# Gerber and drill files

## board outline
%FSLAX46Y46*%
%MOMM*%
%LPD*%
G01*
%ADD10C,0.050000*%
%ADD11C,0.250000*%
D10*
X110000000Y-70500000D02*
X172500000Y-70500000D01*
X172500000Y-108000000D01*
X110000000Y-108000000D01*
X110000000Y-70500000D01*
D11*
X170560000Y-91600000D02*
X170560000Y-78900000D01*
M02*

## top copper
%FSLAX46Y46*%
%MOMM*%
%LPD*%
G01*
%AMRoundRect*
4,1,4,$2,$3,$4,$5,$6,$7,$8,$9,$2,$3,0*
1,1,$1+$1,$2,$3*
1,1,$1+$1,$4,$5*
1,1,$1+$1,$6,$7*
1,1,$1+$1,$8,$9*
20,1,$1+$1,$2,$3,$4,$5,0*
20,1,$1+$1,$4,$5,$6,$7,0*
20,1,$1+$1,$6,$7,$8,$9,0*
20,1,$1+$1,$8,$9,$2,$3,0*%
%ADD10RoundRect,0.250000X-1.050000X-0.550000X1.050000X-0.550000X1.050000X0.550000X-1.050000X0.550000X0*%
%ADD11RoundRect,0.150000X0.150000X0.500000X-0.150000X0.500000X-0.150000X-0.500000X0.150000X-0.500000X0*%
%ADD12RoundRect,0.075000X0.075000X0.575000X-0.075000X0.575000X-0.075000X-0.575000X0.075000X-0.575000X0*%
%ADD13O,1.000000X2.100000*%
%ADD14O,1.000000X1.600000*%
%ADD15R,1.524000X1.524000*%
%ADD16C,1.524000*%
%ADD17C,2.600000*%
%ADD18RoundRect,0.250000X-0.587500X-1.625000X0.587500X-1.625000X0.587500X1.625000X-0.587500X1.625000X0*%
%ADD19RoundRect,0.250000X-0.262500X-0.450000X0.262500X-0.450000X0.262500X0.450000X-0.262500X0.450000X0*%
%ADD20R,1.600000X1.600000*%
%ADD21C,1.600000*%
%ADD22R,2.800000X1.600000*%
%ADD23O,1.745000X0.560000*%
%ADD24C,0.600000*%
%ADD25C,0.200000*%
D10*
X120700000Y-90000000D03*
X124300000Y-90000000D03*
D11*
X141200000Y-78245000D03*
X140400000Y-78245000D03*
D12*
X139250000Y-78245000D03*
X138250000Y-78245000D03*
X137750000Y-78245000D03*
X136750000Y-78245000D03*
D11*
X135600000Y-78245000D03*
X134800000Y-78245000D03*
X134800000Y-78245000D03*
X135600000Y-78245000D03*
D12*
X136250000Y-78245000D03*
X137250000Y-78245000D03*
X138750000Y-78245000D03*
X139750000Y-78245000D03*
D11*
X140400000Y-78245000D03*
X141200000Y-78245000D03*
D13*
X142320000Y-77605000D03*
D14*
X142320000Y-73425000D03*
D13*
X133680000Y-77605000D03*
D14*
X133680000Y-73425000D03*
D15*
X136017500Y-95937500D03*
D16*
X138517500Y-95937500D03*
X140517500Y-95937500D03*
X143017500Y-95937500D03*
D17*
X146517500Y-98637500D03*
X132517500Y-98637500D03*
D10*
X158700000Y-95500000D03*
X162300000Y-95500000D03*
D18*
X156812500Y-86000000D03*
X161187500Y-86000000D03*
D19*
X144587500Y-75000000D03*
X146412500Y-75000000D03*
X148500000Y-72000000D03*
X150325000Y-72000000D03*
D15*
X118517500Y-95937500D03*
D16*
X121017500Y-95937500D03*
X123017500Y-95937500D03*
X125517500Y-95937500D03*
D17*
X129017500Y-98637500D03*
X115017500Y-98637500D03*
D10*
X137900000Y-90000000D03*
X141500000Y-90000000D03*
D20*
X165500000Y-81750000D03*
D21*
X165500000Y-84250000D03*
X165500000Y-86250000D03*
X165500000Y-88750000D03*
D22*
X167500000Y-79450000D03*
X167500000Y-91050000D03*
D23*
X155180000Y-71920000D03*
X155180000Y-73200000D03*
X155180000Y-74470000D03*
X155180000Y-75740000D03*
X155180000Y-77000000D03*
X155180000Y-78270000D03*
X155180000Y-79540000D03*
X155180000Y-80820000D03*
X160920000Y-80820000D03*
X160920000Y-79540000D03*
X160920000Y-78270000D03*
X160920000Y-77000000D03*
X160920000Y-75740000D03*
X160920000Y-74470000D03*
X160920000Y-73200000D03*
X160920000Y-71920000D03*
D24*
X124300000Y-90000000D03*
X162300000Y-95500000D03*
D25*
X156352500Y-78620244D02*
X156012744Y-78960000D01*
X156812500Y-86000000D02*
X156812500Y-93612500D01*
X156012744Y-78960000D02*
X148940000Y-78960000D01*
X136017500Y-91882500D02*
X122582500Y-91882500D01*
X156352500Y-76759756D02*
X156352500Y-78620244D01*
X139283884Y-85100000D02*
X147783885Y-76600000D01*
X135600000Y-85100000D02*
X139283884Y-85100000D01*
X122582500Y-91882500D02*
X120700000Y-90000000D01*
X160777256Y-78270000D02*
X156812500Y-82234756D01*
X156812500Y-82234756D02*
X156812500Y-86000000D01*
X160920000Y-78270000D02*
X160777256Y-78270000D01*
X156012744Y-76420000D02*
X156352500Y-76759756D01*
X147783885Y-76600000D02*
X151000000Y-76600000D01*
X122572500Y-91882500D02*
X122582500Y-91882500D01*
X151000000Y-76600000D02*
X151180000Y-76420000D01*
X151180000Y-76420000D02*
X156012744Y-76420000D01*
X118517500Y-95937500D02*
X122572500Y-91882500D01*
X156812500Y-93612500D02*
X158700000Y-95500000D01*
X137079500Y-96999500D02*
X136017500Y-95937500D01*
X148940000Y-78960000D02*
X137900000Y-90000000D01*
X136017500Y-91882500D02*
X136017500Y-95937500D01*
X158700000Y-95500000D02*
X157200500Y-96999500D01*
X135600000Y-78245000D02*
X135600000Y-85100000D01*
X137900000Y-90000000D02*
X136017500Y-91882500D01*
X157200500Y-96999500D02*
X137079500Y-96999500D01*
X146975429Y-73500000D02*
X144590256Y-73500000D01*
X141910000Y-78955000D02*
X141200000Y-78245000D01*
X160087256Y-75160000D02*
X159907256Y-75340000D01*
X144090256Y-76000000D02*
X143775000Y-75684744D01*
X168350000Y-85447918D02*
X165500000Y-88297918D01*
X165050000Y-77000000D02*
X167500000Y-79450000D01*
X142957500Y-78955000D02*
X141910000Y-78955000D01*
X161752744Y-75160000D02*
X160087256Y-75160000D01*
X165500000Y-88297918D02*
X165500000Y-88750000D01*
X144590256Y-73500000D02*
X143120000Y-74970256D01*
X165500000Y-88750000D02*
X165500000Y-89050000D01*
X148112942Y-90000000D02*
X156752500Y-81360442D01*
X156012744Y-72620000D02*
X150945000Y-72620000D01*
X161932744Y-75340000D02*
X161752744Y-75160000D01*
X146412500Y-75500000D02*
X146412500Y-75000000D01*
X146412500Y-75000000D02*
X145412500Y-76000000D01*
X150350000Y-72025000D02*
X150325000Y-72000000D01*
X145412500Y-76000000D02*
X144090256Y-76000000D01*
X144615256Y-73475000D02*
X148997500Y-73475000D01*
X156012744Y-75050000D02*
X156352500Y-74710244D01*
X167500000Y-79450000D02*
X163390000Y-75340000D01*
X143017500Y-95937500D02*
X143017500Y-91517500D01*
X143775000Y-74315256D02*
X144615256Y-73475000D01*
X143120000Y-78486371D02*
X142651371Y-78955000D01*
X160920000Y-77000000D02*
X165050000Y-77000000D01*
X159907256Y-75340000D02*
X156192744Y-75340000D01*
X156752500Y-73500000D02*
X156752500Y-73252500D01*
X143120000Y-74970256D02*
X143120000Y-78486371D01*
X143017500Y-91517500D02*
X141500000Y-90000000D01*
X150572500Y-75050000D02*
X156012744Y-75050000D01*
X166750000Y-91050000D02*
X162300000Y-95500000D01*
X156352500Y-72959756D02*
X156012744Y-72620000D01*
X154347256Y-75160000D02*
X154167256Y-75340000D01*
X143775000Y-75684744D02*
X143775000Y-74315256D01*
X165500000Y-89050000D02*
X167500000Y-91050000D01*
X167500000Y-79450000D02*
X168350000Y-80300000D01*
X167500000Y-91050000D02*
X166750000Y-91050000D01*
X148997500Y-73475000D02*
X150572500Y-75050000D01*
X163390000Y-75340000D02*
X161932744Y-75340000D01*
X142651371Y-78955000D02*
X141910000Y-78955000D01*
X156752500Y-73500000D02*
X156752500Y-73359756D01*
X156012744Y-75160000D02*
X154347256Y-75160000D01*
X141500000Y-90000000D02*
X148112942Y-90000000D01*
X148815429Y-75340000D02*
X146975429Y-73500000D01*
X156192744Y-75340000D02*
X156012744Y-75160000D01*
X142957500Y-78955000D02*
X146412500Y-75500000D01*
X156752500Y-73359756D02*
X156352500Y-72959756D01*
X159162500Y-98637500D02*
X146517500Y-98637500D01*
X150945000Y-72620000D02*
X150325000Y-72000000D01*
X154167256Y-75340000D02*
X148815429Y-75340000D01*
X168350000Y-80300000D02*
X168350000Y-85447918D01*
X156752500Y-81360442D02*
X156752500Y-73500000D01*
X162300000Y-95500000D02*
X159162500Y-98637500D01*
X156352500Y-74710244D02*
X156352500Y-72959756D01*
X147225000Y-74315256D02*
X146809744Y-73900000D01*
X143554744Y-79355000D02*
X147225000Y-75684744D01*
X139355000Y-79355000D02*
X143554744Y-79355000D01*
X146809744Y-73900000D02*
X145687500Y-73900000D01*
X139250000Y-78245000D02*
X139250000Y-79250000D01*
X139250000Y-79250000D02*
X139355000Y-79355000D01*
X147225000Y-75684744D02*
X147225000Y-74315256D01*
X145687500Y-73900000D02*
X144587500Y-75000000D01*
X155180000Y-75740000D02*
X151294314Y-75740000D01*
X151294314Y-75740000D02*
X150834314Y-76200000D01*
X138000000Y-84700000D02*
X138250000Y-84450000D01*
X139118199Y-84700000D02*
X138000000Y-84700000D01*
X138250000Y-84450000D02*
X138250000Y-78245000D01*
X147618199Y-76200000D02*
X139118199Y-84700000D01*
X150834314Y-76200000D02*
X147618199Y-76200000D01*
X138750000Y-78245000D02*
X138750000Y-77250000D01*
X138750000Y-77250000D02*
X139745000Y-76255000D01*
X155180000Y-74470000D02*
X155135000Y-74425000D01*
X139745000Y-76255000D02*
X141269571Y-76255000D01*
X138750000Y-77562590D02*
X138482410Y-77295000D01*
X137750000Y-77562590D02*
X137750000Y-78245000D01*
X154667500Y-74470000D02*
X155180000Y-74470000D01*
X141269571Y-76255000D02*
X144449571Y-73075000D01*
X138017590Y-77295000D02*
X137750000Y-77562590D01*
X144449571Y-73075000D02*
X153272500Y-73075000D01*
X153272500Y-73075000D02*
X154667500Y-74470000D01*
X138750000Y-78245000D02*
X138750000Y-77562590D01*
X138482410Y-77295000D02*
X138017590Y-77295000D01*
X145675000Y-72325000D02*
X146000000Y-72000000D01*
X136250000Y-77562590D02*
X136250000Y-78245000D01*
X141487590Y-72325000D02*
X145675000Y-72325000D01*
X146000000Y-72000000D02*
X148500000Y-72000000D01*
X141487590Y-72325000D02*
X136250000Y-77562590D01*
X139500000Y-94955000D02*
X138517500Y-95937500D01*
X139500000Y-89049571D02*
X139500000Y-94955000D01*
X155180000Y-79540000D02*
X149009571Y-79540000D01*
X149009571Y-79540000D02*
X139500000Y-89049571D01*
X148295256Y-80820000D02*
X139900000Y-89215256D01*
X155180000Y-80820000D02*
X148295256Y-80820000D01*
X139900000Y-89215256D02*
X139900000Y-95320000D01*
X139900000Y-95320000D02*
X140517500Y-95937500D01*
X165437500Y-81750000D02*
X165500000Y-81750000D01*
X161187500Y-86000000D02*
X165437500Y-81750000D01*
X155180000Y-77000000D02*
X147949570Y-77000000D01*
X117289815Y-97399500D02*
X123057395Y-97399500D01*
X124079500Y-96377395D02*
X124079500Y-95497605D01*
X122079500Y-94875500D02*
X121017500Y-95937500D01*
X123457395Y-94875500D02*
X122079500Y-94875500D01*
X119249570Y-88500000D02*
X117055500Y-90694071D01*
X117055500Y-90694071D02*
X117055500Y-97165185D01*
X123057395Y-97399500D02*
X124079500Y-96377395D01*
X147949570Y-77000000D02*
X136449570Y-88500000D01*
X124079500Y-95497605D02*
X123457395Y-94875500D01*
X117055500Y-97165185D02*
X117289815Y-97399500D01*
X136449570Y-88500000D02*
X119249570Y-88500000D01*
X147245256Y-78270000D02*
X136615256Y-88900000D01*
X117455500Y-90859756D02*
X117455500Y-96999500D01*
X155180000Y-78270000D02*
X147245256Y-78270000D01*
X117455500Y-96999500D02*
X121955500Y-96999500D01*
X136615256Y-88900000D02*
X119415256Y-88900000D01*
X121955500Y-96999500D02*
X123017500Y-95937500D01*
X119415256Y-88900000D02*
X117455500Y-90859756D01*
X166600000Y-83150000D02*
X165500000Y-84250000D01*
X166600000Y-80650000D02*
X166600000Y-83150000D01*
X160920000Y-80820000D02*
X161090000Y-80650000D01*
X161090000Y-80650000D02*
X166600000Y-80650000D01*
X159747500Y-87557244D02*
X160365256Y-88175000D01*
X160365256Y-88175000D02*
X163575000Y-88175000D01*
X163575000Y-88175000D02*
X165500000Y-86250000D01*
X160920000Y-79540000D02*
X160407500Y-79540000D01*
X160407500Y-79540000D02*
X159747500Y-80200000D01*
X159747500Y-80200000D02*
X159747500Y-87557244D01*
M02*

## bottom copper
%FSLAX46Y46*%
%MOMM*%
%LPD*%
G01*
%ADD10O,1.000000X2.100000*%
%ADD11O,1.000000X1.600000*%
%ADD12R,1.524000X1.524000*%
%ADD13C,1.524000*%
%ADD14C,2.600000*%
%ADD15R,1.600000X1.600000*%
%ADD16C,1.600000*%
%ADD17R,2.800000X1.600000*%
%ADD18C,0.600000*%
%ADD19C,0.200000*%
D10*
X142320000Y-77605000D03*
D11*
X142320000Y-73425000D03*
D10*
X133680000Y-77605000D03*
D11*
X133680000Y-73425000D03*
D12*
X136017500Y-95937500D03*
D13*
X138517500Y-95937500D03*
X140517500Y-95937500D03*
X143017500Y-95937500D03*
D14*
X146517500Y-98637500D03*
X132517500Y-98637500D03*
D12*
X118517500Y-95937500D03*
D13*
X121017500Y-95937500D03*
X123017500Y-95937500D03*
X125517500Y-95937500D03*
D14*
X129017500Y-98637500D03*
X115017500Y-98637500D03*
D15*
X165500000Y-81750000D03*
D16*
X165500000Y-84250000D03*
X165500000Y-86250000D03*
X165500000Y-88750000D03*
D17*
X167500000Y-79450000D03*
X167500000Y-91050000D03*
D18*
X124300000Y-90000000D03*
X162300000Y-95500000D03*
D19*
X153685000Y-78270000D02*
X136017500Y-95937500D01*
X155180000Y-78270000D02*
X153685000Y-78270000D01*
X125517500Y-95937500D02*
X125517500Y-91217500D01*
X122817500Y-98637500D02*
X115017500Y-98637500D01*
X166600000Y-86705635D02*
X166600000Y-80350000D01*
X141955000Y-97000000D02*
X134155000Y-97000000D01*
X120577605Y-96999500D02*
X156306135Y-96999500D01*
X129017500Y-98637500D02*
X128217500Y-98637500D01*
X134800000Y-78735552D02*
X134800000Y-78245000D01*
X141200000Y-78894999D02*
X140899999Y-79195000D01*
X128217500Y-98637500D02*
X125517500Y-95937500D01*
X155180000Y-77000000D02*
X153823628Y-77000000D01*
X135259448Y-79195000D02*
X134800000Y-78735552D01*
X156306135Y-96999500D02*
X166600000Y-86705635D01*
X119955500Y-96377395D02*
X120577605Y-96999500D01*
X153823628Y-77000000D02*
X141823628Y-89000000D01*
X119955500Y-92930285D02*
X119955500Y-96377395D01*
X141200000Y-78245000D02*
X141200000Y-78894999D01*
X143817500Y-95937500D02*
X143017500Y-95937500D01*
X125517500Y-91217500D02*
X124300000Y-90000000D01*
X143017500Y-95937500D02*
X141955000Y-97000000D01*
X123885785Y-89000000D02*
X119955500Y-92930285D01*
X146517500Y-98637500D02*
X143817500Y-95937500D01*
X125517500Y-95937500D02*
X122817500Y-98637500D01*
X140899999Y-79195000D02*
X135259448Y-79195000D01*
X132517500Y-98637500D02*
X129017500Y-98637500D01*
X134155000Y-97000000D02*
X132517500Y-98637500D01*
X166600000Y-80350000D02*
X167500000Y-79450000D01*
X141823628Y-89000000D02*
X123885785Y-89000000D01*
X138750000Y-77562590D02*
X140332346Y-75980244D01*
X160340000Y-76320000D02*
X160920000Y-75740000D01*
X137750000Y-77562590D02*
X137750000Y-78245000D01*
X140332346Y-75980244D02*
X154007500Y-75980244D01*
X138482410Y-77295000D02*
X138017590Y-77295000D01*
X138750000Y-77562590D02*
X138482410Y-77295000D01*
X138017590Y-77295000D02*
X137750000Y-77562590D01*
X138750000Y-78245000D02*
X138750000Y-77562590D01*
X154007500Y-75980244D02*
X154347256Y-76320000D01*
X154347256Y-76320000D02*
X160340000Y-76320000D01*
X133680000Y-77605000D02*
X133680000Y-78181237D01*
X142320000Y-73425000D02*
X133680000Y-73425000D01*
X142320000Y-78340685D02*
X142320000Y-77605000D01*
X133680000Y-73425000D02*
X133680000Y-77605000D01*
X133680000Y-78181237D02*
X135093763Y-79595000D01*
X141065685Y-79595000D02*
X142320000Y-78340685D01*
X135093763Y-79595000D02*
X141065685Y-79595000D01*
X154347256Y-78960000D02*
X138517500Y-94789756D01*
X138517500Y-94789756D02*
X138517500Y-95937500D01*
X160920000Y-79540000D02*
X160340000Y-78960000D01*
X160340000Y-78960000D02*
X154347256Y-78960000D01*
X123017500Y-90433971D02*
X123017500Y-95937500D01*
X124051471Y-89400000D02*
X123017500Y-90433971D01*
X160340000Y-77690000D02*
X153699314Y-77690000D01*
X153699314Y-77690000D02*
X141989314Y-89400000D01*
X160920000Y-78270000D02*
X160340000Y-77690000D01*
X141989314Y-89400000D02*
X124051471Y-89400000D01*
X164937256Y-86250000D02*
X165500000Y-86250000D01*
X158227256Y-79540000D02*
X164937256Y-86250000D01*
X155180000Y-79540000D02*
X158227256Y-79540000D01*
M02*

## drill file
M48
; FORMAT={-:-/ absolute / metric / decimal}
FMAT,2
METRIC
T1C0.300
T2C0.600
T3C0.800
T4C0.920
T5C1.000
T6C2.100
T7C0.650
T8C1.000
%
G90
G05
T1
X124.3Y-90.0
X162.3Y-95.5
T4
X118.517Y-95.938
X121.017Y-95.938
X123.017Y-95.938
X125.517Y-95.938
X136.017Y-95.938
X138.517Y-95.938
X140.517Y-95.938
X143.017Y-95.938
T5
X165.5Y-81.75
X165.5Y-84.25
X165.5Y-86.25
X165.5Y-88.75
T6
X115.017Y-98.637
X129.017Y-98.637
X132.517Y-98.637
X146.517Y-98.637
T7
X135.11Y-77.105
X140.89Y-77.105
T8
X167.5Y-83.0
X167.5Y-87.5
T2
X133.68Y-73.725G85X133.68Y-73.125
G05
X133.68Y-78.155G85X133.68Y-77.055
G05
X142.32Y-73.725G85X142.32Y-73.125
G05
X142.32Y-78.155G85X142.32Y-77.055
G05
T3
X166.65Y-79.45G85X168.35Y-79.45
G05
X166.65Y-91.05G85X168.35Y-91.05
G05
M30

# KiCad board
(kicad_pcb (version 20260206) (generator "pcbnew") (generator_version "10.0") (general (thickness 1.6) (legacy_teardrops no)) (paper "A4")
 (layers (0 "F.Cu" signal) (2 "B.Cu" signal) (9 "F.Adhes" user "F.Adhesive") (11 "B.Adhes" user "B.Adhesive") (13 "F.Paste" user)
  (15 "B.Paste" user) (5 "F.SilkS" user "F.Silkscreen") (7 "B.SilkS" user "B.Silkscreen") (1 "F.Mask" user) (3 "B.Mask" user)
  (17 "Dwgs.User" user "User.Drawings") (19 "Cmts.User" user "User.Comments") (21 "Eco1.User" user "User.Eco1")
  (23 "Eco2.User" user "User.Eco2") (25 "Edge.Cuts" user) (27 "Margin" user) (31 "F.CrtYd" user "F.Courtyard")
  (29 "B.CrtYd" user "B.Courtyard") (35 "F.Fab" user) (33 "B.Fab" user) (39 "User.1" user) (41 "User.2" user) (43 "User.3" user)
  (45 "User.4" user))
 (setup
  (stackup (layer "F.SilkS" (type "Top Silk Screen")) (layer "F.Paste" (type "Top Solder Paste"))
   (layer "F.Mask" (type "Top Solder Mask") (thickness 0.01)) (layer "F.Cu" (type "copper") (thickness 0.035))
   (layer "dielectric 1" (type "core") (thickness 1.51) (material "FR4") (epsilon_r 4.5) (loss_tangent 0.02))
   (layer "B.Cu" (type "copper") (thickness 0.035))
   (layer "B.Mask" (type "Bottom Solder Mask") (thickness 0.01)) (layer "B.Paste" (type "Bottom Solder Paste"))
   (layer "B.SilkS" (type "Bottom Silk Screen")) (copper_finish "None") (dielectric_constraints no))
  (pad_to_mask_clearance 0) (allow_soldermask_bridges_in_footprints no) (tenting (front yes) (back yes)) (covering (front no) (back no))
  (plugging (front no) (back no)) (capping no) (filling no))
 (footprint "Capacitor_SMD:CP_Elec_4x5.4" (layer "F.Cu") (at 122.5 90)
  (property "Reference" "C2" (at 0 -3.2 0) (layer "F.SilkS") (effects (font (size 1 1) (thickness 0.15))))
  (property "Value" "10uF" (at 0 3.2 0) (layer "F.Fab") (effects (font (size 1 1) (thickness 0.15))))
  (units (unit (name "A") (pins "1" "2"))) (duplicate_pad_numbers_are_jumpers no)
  (pad "1" smd roundrect (at -1.8 0) (size 2.6 1.6) (layers "F.Cu" "F.Mask" "F.Paste") (roundrect_rratio 0.15625) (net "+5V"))
  (pad "2" smd roundrect (at 1.8 0) (size 2.6 1.6) (layers "F.Cu" "F.Mask" "F.Paste") (roundrect_rratio 0.15625) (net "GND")))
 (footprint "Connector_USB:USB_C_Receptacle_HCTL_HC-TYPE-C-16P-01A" (layer "F.Cu") (at 138 74.5 180)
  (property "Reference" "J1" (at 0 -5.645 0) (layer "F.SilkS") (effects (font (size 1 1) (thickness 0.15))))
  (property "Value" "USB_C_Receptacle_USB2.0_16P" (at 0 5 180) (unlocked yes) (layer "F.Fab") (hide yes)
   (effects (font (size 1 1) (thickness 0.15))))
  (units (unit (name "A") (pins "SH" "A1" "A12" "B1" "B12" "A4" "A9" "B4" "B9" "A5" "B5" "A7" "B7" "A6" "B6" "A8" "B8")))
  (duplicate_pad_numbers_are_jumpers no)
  (pad "" np_thru_hole circle (at -2.89 -2.605 180) (size 0.65 0.65) (drill 0.65) (layers "*.Mask"))
  (pad "" np_thru_hole circle (at 2.89 -2.605 180) (size 0.65 0.65) (drill 0.65) (layers "*.Mask"))
  (pad "A1" smd roundrect (at -3.2 -3.745 180) (size 0.6 1.3) (layers "F.Cu" "F.Mask" "F.Paste") (roundrect_rratio 0.25) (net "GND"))
  (pad "A4" smd roundrect (at -2.4 -3.745 180) (size 0.6 1.3) (layers "F.Cu" "F.Mask" "F.Paste") (roundrect_rratio 0.25) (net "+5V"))
  (pad "A5" smd roundrect (at -1.25 -3.745 180) (size 0.3 1.3) (layers "F.Cu" "F.Mask" "F.Paste") (roundrect_rratio 0.25)
   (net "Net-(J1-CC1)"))
  (pad "A6" smd roundrect (at -0.25 -3.745 180) (size 0.3 1.3) (layers "F.Cu" "F.Mask" "F.Paste") (roundrect_rratio 0.25)
   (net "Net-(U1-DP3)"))
  (pad "A7" smd roundrect (at 0.25 -3.745 180) (size 0.3 1.3) (layers "F.Cu" "F.Mask" "F.Paste") (roundrect_rratio 0.25)
   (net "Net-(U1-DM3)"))
  (pad "A8" smd roundrect (at 1.25 -3.745 180) (size 0.3 1.3) (layers "F.Cu" "F.Mask" "F.Paste") (roundrect_rratio 0.25)
   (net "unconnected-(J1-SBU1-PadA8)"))
  (pad "A9" smd roundrect (at 2.4 -3.745 180) (size 0.6 1.3) (layers "F.Cu" "F.Mask" "F.Paste") (roundrect_rratio 0.25) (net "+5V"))
  (pad "A12" smd roundrect (at 3.2 -3.745 180) (size 0.6 1.3) (layers "F.Cu" "F.Mask" "F.Paste") (roundrect_rratio 0.25) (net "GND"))
  (pad "B1" smd roundrect (at 3.2 -3.745 180) (size 0.6 1.3) (layers "F.Cu" "F.Mask" "F.Paste") (roundrect_rratio 0.25) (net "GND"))
  (pad "B4" smd roundrect (at 2.4 -3.745 180) (size 0.6 1.3) (layers "F.Cu" "F.Mask" "F.Paste") (roundrect_rratio 0.25) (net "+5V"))
  (pad "B5" smd roundrect (at 1.75 -3.745 180) (size 0.3 1.3) (layers "F.Cu" "F.Mask" "F.Paste") (roundrect_rratio 0.25)
   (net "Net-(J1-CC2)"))
  (pad "B6" smd roundrect (at 0.75 -3.745 180) (size 0.3 1.3) (layers "F.Cu" "F.Mask" "F.Paste") (roundrect_rratio 0.25)
   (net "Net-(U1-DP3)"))
  (pad "B7" smd roundrect (at -0.75 -3.745 180) (size 0.3 1.3) (layers "F.Cu" "F.Mask" "F.Paste") (roundrect_rratio 0.25)
   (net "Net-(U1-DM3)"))
  (pad "B8" smd roundrect (at -1.75 -3.745 180) (size 0.3 1.3) (layers "F.Cu" "F.Mask" "F.Paste") (roundrect_rratio 0.25)
   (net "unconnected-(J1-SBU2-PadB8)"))
  (pad "B9" smd roundrect (at -2.4 -3.745 180) (size 0.6 1.3) (layers "F.Cu" "F.Mask" "F.Paste") (roundrect_rratio 0.25) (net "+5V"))
  (pad "B12" smd roundrect (at -3.2 -3.745 180) (size 0.6 1.3) (layers "F.Cu" "F.Mask" "F.Paste") (roundrect_rratio 0.25) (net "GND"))
  (pad "SH" thru_hole oval (at -4.32 -3.105 180) (size 1 2.1) (drill oval 0.6 1.7) (layers "*.Cu" "*.Mask") (remove_unused_layers no)
   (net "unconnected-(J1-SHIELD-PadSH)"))
  (pad "SH" thru_hole oval (at -4.32 1.075 180) (size 1 1.6) (drill oval 0.6 1.2) (layers "*.Cu" "*.Mask") (remove_unused_layers no)
   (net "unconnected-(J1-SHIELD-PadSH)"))
  (pad "SH" thru_hole oval (at 4.32 -3.105 180) (size 1 2.1) (drill oval 0.6 1.7) (layers "*.Cu" "*.Mask") (remove_unused_layers no)
   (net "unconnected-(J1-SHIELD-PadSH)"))
  (pad "SH" thru_hole oval (at 4.32 1.075 180) (size 1 1.6) (drill oval 0.6 1.2) (layers "*.Cu" "*.Mask") (remove_unused_layers no)
   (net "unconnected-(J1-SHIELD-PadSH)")))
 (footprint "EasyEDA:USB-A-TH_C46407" (layer "F.Cu") (at 139.5175 97.2875)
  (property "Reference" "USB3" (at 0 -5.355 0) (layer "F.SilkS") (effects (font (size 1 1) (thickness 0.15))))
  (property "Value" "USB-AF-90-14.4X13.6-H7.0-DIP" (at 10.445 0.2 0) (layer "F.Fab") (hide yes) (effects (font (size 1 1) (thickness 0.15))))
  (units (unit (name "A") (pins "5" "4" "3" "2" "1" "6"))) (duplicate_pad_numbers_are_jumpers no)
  (pad "1" thru_hole rect (at -3.5 -1.35) (size 1.524 1.524) (drill 0.919988) (layers "*.Cu" "*.Mask") (remove_unused_layers no) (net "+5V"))
  (pad "2" thru_hole circle (at -1 -1.35) (size 1.524 1.524) (drill 0.919988) (layers "*.Cu" "*.Mask") (remove_unused_layers no)
   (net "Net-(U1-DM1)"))
  (pad "3" thru_hole circle (at 1 -1.35) (size 1.524 1.524) (drill 0.919988) (layers "*.Cu" "*.Mask") (remove_unused_layers no)
   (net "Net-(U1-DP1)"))
  (pad "4" thru_hole circle (at 3.5 -1.35) (size 1.524 1.524) (drill 0.919988) (layers "*.Cu" "*.Mask") (remove_unused_layers no)
   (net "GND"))
  (pad "5" thru_hole circle (at 7 1.35) (size 2.6 2.6) (drill 2.100022) (layers "*.Cu" "*.Mask") (remove_unused_layers no) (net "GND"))
  (pad "6" thru_hole circle (at -7 1.35) (size 2.6 2.6) (drill 2.100022) (layers "*.Cu" "*.Mask") (remove_unused_layers no) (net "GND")))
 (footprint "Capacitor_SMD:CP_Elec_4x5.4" (layer "F.Cu") (at 160.5 95.5)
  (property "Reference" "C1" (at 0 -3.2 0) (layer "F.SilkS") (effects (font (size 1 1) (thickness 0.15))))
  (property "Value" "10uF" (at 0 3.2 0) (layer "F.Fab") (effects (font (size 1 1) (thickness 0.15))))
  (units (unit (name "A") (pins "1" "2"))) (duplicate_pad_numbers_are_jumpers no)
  (pad "1" smd roundrect (at -1.8 0) (size 2.6 1.6) (layers "F.Cu" "F.Mask" "F.Paste") (roundrect_rratio 0.15625) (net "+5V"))
  (pad "2" smd roundrect (at 1.8 0) (size 2.6 1.6) (layers "F.Cu" "F.Mask" "F.Paste") (roundrect_rratio 0.15625) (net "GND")))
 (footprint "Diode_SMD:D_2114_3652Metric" (layer "F.Cu") (at 159 86)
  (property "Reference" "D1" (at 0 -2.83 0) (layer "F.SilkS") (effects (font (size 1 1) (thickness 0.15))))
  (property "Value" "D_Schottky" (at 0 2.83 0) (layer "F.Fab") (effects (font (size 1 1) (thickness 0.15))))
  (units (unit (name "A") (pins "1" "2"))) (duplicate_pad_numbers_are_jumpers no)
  (pad "1" smd roundrect (at -2.1875 0) (size 1.675 3.75) (layers "F.Cu" "F.Mask" "F.Paste") (roundrect_rratio 0.149254) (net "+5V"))
  (pad "2" smd roundrect (at 2.1875 0) (size 1.675 3.75) (layers "F.Cu" "F.Mask" "F.Paste") (roundrect_rratio 0.149254) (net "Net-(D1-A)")))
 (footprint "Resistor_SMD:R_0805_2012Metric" (layer "F.Cu") (at 145.5 75)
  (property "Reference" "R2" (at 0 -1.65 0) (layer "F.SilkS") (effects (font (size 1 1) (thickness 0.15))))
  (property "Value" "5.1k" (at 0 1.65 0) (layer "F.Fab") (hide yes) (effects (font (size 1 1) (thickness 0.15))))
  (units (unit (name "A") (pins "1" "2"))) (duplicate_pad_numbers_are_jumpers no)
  (pad "1" smd roundrect (at -0.9125 0) (size 1.025 1.4) (layers "F.Cu" "F.Mask" "F.Paste") (roundrect_rratio 0.243902) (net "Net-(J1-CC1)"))
  (pad "2" smd roundrect (at 0.9125 0) (size 1.025 1.4) (layers "F.Cu" "F.Mask" "F.Paste") (roundrect_rratio 0.243902) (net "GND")))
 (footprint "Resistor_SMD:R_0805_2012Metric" (layer "F.Cu") (at 149.4125 72)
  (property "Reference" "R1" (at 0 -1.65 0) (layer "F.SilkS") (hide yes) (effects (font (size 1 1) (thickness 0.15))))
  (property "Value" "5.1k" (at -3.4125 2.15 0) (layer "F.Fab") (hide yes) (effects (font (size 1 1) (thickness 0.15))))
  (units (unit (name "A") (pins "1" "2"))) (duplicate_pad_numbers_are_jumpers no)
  (pad "1" smd roundrect (at -0.9125 0) (size 1.025 1.4) (layers "F.Cu" "F.Mask" "F.Paste") (roundrect_rratio 0.243902) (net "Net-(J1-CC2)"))
  (pad "2" smd roundrect (at 0.9125 0) (size 1.025 1.4) (layers "F.Cu" "F.Mask" "F.Paste") (roundrect_rratio 0.243902) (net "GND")))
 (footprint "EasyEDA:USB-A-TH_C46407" (layer "F.Cu") (at 122.0175 97.2875)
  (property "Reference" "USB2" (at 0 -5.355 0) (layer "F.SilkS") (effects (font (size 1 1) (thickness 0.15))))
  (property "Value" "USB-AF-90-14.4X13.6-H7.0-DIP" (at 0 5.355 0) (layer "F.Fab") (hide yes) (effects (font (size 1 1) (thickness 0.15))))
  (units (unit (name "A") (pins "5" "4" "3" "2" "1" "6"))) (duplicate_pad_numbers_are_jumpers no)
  (pad "1" thru_hole rect (at -3.5 -1.35) (size 1.524 1.524) (drill 0.919988) (layers "*.Cu" "*.Mask") (remove_unused_layers no) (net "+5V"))
  (pad "2" thru_hole circle (at -1 -1.35) (size 1.524 1.524) (drill 0.919988) (layers "*.Cu" "*.Mask") (remove_unused_layers no)
   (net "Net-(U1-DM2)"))
  (pad "3" thru_hole circle (at 1 -1.35) (size 1.524 1.524) (drill 0.919988) (layers "*.Cu" "*.Mask") (remove_unused_layers no)
   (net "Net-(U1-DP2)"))
  (pad "4" thru_hole circle (at 3.5 -1.35) (size 1.524 1.524) (drill 0.919988) (layers "*.Cu" "*.Mask") (remove_unused_layers no)
   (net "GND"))
  (pad "5" thru_hole circle (at 7 1.35) (size 2.6 2.6) (drill 2.100022) (layers "*.Cu" "*.Mask") (remove_unused_layers no) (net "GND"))
  (pad "6" thru_hole circle (at -7 1.35) (size 2.6 2.6) (drill 2.100022) (layers "*.Cu" "*.Mask") (remove_unused_layers no) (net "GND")))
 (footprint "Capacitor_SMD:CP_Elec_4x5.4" (layer "F.Cu") (at 139.7 90)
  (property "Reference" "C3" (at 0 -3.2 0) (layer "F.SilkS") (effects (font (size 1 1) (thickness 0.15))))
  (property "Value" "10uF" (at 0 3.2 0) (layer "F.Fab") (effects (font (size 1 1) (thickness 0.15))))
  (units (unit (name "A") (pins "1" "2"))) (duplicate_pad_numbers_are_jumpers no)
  (pad "1" smd roundrect (at -1.8 0) (size 2.6 1.6) (layers "F.Cu" "F.Mask" "F.Paste") (roundrect_rratio 0.15625) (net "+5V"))
  (pad "2" smd roundrect (at 1.8 0) (size 2.6 1.6) (layers "F.Cu" "F.Mask" "F.Paste") (roundrect_rratio 0.15625) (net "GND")))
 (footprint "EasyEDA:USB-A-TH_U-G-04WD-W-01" (layer "F.Cu") (at 166.5 85.25 90)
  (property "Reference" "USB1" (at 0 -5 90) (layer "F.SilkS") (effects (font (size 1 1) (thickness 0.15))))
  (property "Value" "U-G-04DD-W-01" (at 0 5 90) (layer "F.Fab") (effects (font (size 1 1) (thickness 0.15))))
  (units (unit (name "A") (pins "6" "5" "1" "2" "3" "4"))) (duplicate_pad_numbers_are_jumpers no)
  (fp_line (start -6.35 4.06) (end 6.35 4.06) (stroke (width 0.25) (type solid)) (layer "Edge.Cuts"))
  (pad "" np_thru_hole circle (at -2.25 1 90) (size 1 1) (drill 1) (layers "*.Cu" "*.Mask"))
  (pad "" np_thru_hole circle (at 2.25 1 90) (size 1 1) (drill 1) (layers "*.Cu" "*.Mask"))
  (pad "1" thru_hole rect (at 3.5 -1 90) (size 1.6 1.6) (drill 0.999998) (layers "*.Cu" "*.Mask") (remove_unused_layers no)
   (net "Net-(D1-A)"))
  (pad "2" thru_hole circle (at 1 -1 90) (size 1.6 1.6) (drill 0.999998) (layers "*.Cu" "*.Mask") (remove_unused_layers no)
   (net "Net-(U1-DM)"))
  (pad "3" thru_hole circle (at -1 -1 90) (size 1.6 1.6) (drill 0.999998) (layers "*.Cu" "*.Mask") (remove_unused_layers no)
   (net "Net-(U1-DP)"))
  (pad "4" thru_hole circle (at -3.5 -1 90) (size 1.6 1.6) (drill 0.999998) (layers "*.Cu" "*.Mask") (remove_unused_layers no) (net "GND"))
  (pad "5" thru_hole rect (at 5.8 1 90) (size 1.6 2.8) (drill oval 0.799998 2.499995) (layers "*.Cu" "*.Mask") (remove_unused_layers no)
   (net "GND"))
  (pad "6" thru_hole rect (at -5.8 1 90) (size 1.6 2.8) (drill oval 0.799998 2.499995) (layers "*.Cu" "*.Mask") (remove_unused_layers no)
   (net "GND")))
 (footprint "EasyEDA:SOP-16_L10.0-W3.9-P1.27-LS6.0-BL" (layer "F.Cu") (at 158.05 76.37 -90)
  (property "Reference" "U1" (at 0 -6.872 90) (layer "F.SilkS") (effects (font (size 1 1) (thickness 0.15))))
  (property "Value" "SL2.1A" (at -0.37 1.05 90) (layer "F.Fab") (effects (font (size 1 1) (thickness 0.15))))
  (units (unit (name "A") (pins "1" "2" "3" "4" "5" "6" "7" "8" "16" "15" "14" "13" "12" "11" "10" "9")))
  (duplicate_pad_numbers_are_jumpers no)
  (pad "1" smd oval (at -4.45 2.87 270) (size 0.56 1.745) (layers "F.Cu" "F.Mask" "F.Paste") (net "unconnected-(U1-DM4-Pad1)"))
  (pad "2" smd oval (at -3.17 2.87 270) (size 0.56 1.745) (layers "F.Cu" "F.Mask" "F.Paste") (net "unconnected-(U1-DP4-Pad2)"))
  (pad "3" smd oval (at -1.9 2.87 270) (size 0.56 1.745) (layers "F.Cu" "F.Mask" "F.Paste") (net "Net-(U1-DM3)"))
  (pad "4" smd oval (at -0.63 2.87 270) (size 0.56 1.745) (layers "F.Cu" "F.Mask" "F.Paste") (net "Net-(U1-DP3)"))
  (pad "5" smd oval (at 0.63 2.87 270) (size 0.56 1.745) (layers "F.Cu" "F.Mask" "F.Paste") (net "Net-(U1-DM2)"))
  (pad "6" smd oval (at 1.9 2.87 270) (size 0.56 1.745) (layers "F.Cu" "F.Mask" "F.Paste") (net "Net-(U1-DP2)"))
  (pad "7" smd oval (at 3.17 2.87 270) (size 0.56 1.745) (layers "F.Cu" "F.Mask" "F.Paste") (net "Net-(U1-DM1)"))
  (pad "8" smd oval (at 4.45 2.87 270) (size 0.56 1.745) (layers "F.Cu" "F.Mask" "F.Paste") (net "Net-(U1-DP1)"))
  (pad "9" smd oval (at 4.45 -2.87 270) (size 0.56 1.745) (layers "F.Cu" "F.Mask" "F.Paste") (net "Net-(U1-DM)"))
  (pad "10" smd oval (at 3.17 -2.87 270) (size 0.56 1.745) (layers "F.Cu" "F.Mask" "F.Paste") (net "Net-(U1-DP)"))
  (pad "11" smd oval (at 1.9 -2.87 270) (size 0.56 1.745) (layers "F.Cu" "F.Mask" "F.Paste") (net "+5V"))
  (pad "12" smd oval (at 0.63 -2.87 270) (size 0.56 1.745) (layers "F.Cu" "F.Mask" "F.Paste") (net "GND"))
  (pad "13" smd oval (at -0.63 -2.87 270) (size 0.56 1.745) (layers "F.Cu" "F.Mask" "F.Paste") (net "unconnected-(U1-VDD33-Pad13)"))
  (pad "14" smd oval (at -1.9 -2.87 270) (size 0.56 1.745) (layers "F.Cu" "F.Mask" "F.Paste") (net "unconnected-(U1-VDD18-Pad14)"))
  (pad "15" smd oval (at -3.17 -2.87 270) (size 0.56 1.745) (layers "F.Cu" "F.Mask" "F.Paste") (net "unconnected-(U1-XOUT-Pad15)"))
  (pad "16" smd oval (at -4.45 -2.87 270) (size 0.56 1.745) (layers "F.Cu" "F.Mask" "F.Paste") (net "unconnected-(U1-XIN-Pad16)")))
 (gr_rect (start 110 70.5) (end 172.5 108) (stroke (width 0.05) (type default)) (fill no) (layer "Edge.Cuts"))
 (segment (start 156.3525 78.620244) (end 156.012744 78.96) (width 0.2) (layer "F.Cu") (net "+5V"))
 (segment (start 156.8125 86) (end 156.8125 93.6125) (width 0.2) (layer "F.Cu") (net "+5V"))
 (segment (start 156.012744 78.96) (end 148.94 78.96) (width 0.2) (layer "F.Cu") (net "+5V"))
 (segment (start 136.0175 91.8825) (end 122.5825 91.8825) (width 0.2) (layer "F.Cu") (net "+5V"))
 (segment (start 156.3525 76.759756) (end 156.3525 78.620244) (width 0.2) (layer "F.Cu") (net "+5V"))
 (segment (start 139.283884 85.1) (end 147.783885 76.6) (width 0.2) (layer "F.Cu") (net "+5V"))
 (segment (start 135.6 85.1) (end 139.283884 85.1) (width 0.2) (layer "F.Cu") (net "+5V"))
 (segment (start 122.5825 91.8825) (end 120.7 90) (width 0.2) (layer "F.Cu") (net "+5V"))
 (segment (start 160.777256 78.27) (end 156.8125 82.234756) (width 0.2) (layer "F.Cu") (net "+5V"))
 (segment (start 156.8125 82.234756) (end 156.8125 86) (width 0.2) (layer "F.Cu") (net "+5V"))
 (segment (start 160.92 78.27) (end 160.777256 78.27) (width 0.2) (layer "F.Cu") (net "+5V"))
 (segment (start 156.012744 76.42) (end 156.3525 76.759756) (width 0.2) (layer "F.Cu") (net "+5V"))
 (segment (start 147.783885 76.6) (end 151 76.6) (width 0.2) (layer "F.Cu") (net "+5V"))
 (segment (start 122.5725 91.8825) (end 122.5825 91.8825) (width 0.2) (layer "F.Cu") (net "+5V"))
 (segment (start 151 76.6) (end 151.18 76.42) (width 0.2) (layer "F.Cu") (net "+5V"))
 (segment (start 151.18 76.42) (end 156.012744 76.42) (width 0.2) (layer "F.Cu") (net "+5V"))
 (segment (start 118.5175 95.9375) (end 122.5725 91.8825) (width 0.2) (layer "F.Cu") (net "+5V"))
 (segment (start 156.8125 93.6125) (end 158.7 95.5) (width 0.2) (layer "F.Cu") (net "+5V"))
 (segment (start 137.0795 96.9995) (end 136.0175 95.9375) (width 0.2) (layer "F.Cu") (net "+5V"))
 (segment (start 148.94 78.96) (end 137.9 90) (width 0.2) (layer "F.Cu") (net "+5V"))
 (segment (start 136.0175 91.8825) (end 136.0175 95.9375) (width 0.2) (layer "F.Cu") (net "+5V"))
 (segment (start 158.7 95.5) (end 157.2005 96.9995) (width 0.2) (layer "F.Cu") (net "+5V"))
 (segment (start 135.6 78.245) (end 135.6 85.1) (width 0.2) (layer "F.Cu") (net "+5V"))
 (segment (start 137.9 90) (end 136.0175 91.8825) (width 0.2) (layer "F.Cu") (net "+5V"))
 (segment (start 157.2005 96.9995) (end 137.0795 96.9995) (width 0.2) (layer "F.Cu") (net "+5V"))
 (segment (start 153.685 78.27) (end 136.0175 95.9375) (width 0.2) (layer "B.Cu") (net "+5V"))
 (segment (start 155.18 78.27) (end 153.685 78.27) (width 0.2) (layer "B.Cu") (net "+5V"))
 (segment (start 146.975429 73.5) (end 144.590256 73.5) (width 0.2) (layer "F.Cu") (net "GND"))
 (segment (start 141.91 78.955) (end 141.2 78.245) (width 0.2) (layer "F.Cu") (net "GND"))
 (segment (start 160.087256 75.16) (end 159.907256 75.34) (width 0.2) (layer "F.Cu") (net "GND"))
 (segment (start 144.090256 76) (end 143.775 75.684744) (width 0.2) (layer "F.Cu") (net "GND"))
 (segment (start 168.35 85.447918) (end 165.5 88.297918) (width 0.2) (layer "F.Cu") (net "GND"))
 (segment (start 165.05 77) (end 167.5 79.45) (width 0.2) (layer "F.Cu") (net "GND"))
 (segment (start 142.9575 78.955) (end 141.91 78.955) (width 0.2) (layer "F.Cu") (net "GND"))
 (segment (start 161.752744 75.16) (end 160.087256 75.16) (width 0.2) (layer "F.Cu") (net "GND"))
 (segment (start 165.5 88.297918) (end 165.5 88.75) (width 0.2) (layer "F.Cu") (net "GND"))
 (segment (start 144.590256 73.5) (end 143.12 74.970256) (width 0.2) (layer "F.Cu") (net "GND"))
 (segment (start 165.5 88.75) (end 165.5 89.05) (width 0.2) (layer "F.Cu") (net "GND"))
 (segment (start 148.112942 90) (end 156.7525 81.360442) (width 0.2) (layer "F.Cu") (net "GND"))
 (segment (start 156.012744 72.62) (end 150.945 72.62) (width 0.2) (layer "F.Cu") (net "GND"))
 (segment (start 161.932744 75.34) (end 161.752744 75.16) (width 0.2) (layer "F.Cu") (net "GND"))
 (segment (start 146.4125 75.5) (end 146.4125 75) (width 0.2) (layer "F.Cu") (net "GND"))
 (segment (start 146.4125 75) (end 145.4125 76) (width 0.2) (layer "F.Cu") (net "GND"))
 (segment (start 150.35 72.025) (end 150.325 72) (width 0.2) (layer "F.Cu") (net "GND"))
 (segment (start 145.4125 76) (end 144.090256 76) (width 0.2) (layer "F.Cu") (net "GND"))
 (segment (start 144.615256 73.475) (end 148.9975 73.475) (width 0.2) (layer "F.Cu") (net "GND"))
 (segment (start 156.012744 75.05) (end 156.3525 74.710244) (width 0.2) (layer "F.Cu") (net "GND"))
 (segment (start 167.5 79.45) (end 163.39 75.34) (width 0.2) (layer "F.Cu") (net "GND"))
 (segment (start 143.0175 95.9375) (end 143.0175 91.5175) (width 0.2) (layer "F.Cu") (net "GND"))
 (segment (start 143.775 74.315256) (end 144.615256 73.475) (width 0.2) (layer "F.Cu") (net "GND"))
 (segment (start 143.12 78.486371) (end 142.651371 78.955) (width 0.2) (layer "F.Cu") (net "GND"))
 (segment (start 160.92 77) (end 165.05 77) (width 0.2) (layer "F.Cu") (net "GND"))
 (segment (start 159.907256 75.34) (end 156.192744 75.34) (width 0.2) (layer "F.Cu") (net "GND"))
 (segment (start 156.7525 73.5) (end 156.7525 73.2525) (width 0.2) (layer "F.Cu") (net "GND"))
 (segment (start 143.12 74.970256) (end 143.12 78.486371) (width 0.2) (layer "F.Cu") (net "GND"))
 (segment (start 143.0175 91.5175) (end 141.5 90) (width 0.2) (layer "F.Cu") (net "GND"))
 (segment (start 150.5725 75.05) (end 156.012744 75.05) (width 0.2) (layer "F.Cu") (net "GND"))
 (segment (start 166.75 91.05) (end 162.3 95.5) (width 0.2) (layer "F.Cu") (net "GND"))
 (segment (start 156.3525 72.959756) (end 156.012744 72.62) (width 0.2) (layer "F.Cu") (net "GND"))
 (segment (start 154.347256 75.16) (end 154.167256 75.34) (width 0.2) (layer "F.Cu") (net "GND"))
 (segment (start 143.775 75.684744) (end 143.775 74.315256) (width 0.2) (layer "F.Cu") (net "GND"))
 (segment (start 165.5 89.05) (end 167.5 91.05) (width 0.2) (layer "F.Cu") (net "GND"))
 (segment (start 167.5 79.45) (end 168.35 80.3) (width 0.2) (layer "F.Cu") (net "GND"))
 (segment (start 167.5 91.05) (end 166.75 91.05) (width 0.2) (layer "F.Cu") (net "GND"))
 (segment (start 148.9975 73.475) (end 150.5725 75.05) (width 0.2) (layer "F.Cu") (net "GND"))
 (segment (start 163.39 75.34) (end 161.932744 75.34) (width 0.2) (layer "F.Cu") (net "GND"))
 (segment (start 142.651371 78.955) (end 141.91 78.955) (width 0.2) (layer "F.Cu") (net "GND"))
 (segment (start 156.7525 73.5) (end 156.7525 73.359756) (width 0.2) (layer "F.Cu") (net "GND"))
 (segment (start 156.012744 75.16) (end 154.347256 75.16) (width 0.2) (layer "F.Cu") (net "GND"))
 (segment (start 141.5 90) (end 148.112942 90) (width 0.2) (layer "F.Cu") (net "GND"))
 (segment (start 148.815429 75.34) (end 146.975429 73.5) (width 0.2) (layer "F.Cu") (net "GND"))
 (segment (start 156.192744 75.34) (end 156.012744 75.16) (width 0.2) (layer "F.Cu") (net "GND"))
 (segment (start 142.9575 78.955) (end 146.4125 75.5) (width 0.2) (layer "F.Cu") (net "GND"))
 (segment (start 156.7525 73.359756) (end 156.3525 72.959756) (width 0.2) (layer "F.Cu") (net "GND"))
 (segment (start 159.1625 98.6375) (end 146.5175 98.6375) (width 0.2) (layer "F.Cu") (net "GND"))
 (segment (start 150.945 72.62) (end 150.325 72) (width 0.2) (layer "F.Cu") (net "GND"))
 (segment (start 154.167256 75.34) (end 148.815429 75.34) (width 0.2) (layer "F.Cu") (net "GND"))
 (segment (start 168.35 80.3) (end 168.35 85.447918) (width 0.2) (layer "F.Cu") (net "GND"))
 (segment (start 156.7525 81.360442) (end 156.7525 73.5) (width 0.2) (layer "F.Cu") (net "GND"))
 (segment (start 162.3 95.5) (end 159.1625 98.6375) (width 0.2) (layer "F.Cu") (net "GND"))
 (segment (start 156.3525 74.710244) (end 156.3525 72.959756) (width 0.2) (layer "F.Cu") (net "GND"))
 (via (at 124.3 90) (size 0.6) (drill 0.3) (layers "F.Cu" "B.Cu") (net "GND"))
 (via (at 162.3 95.5) (size 0.6) (drill 0.3) (layers "F.Cu" "B.Cu") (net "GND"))
 (segment (start 125.5175 95.9375) (end 125.5175 91.2175) (width 0.2) (layer "B.Cu") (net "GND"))
 (segment (start 122.8175 98.6375) (end 115.0175 98.6375) (width 0.2) (layer "B.Cu") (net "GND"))
 (segment (start 166.6 86.705635) (end 166.6 80.35) (width 0.2) (layer "B.Cu") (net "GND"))
 (segment (start 141.955 97) (end 134.155 97) (width 0.2) (layer "B.Cu") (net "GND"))
 (segment (start 120.577605 96.9995) (end 156.306135 96.9995) (width 0.2) (layer "B.Cu") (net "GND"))
 (segment (start 129.0175 98.6375) (end 128.2175 98.6375) (width 0.2) (layer "B.Cu") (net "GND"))
 (segment (start 134.8 78.735552) (end 134.8 78.245) (width 0.2) (layer "B.Cu") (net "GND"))
 (segment (start 141.2 78.894999) (end 140.899999 79.195) (width 0.2) (layer "B.Cu") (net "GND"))
 (segment (start 128.2175 98.6375) (end 125.5175 95.9375) (width 0.2) (layer "B.Cu") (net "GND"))
 (segment (start 155.18 77) (end 153.823628 77) (width 0.2) (layer "B.Cu") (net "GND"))
 (segment (start 135.259448 79.195) (end 134.8 78.735552) (width 0.2) (layer "B.Cu") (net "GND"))
 (segment (start 156.306135 96.9995) (end 166.6 86.705635) (width 0.2) (layer "B.Cu") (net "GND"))
 (segment (start 119.9555 96.377395) (end 120.577605 96.9995) (width 0.2) (layer "B.Cu") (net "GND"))
 (segment (start 153.823628 77) (end 141.823628 89) (width 0.2) (layer "B.Cu") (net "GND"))
 (segment (start 119.9555 92.930285) (end 119.9555 96.377395) (width 0.2) (layer "B.Cu") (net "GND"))
 (segment (start 141.2 78.245) (end 141.2 78.894999) (width 0.2) (layer "B.Cu") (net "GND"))
 (segment (start 143.8175 95.9375) (end 143.0175 95.9375) (width 0.2) (layer "B.Cu") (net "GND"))
 (segment (start 125.5175 91.2175) (end 124.3 90) (width 0.2) (layer "B.Cu") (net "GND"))
 (segment (start 143.0175 95.9375) (end 141.955 97) (width 0.2) (layer "B.Cu") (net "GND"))
 (segment (start 123.885785 89) (end 119.9555 92.930285) (width 0.2) (layer "B.Cu") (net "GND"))
 (segment (start 146.5175 98.6375) (end 143.8175 95.9375) (width 0.2) (layer "B.Cu") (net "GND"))
 (segment (start 125.5175 95.9375) (end 122.8175 98.6375) (width 0.2) (layer "B.Cu") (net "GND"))
 (segment (start 140.899999 79.195) (end 135.259448 79.195) (width 0.2) (layer "B.Cu") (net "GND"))
 (segment (start 132.5175 98.6375) (end 129.0175 98.6375) (width 0.2) (layer "B.Cu") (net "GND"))
 (segment (start 134.155 97) (end 132.5175 98.6375) (width 0.2) (layer "B.Cu") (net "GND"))
 (segment (start 166.6 80.35) (end 167.5 79.45) (width 0.2) (layer "B.Cu") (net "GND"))
 (segment (start 141.823628 89) (end 123.885785 89) (width 0.2) (layer "B.Cu") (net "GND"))
 (segment (start 147.225 74.315256) (end 146.809744 73.9) (width 0.2) (layer "F.Cu") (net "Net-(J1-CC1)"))
 (segment (start 143.554744 79.355) (end 147.225 75.684744) (width 0.2) (layer "F.Cu") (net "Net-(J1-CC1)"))
 (segment (start 139.355 79.355) (end 143.554744 79.355) (width 0.2) (layer "F.Cu") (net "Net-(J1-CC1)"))
 (segment (start 146.809744 73.9) (end 145.6875 73.9) (width 0.2) (layer "F.Cu") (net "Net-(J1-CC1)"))
 (segment (start 139.25 78.245) (end 139.25 79.25) (width 0.2) (layer "F.Cu") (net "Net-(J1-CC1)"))
 (segment (start 139.25 79.25) (end 139.355 79.355) (width 0.2) (layer "F.Cu") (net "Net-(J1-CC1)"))
 (segment (start 147.225 75.684744) (end 147.225 74.315256) (width 0.2) (layer "F.Cu") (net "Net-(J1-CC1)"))
 (segment (start 145.6875 73.9) (end 144.5875 75) (width 0.2) (layer "F.Cu") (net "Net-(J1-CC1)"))
 (segment (start 155.18 75.74) (end 151.294314 75.74) (width 0.2) (layer "F.Cu") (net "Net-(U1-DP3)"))
 (segment (start 151.294314 75.74) (end 150.834314 76.2) (width 0.2) (layer "F.Cu") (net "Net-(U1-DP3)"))
 (segment (start 138 84.7) (end 138.25 84.45) (width 0.2) (layer "F.Cu") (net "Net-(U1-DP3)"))
 (segment (start 139.118199 84.7) (end 138 84.7) (width 0.2) (layer "F.Cu") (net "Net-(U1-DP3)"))
 (segment (start 138.25 84.45) (end 138.25 78.245) (width 0.2) (layer "F.Cu") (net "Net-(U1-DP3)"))
 (segment (start 147.618199 76.2) (end 139.118199 84.7) (width 0.2) (layer "F.Cu") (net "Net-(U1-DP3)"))
 (segment (start 150.834314 76.2) (end 147.618199 76.2) (width 0.2) (layer "F.Cu") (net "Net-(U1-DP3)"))
 (segment (start 138.75 77.56259) (end 140.332346 75.980244) (width 0.2) (layer "B.Cu") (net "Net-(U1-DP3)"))
 (segment (start 160.34 76.32) (end 160.92 75.74) (width 0.2) (layer "B.Cu") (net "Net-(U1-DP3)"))
 (segment (start 137.75 77.56259) (end 137.75 78.245) (width 0.2) (layer "B.Cu") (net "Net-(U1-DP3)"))
 (segment (start 140.332346 75.980244) (end 154.0075 75.980244) (width 0.2) (layer "B.Cu") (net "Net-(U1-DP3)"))
 (segment (start 138.48241 77.295) (end 138.01759 77.295) (width 0.2) (layer "B.Cu") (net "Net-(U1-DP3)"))
 (segment (start 138.75 77.56259) (end 138.48241 77.295) (width 0.2) (layer "B.Cu") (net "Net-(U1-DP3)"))
 (segment (start 138.01759 77.295) (end 137.75 77.56259) (width 0.2) (layer "B.Cu") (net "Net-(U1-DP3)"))
 (segment (start 138.75 78.245) (end 138.75 77.56259) (width 0.2) (layer "B.Cu") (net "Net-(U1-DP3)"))
 (segment (start 154.0075 75.980244) (end 154.347256 76.32) (width 0.2) (layer "B.Cu") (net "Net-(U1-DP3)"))
 (segment (start 154.347256 76.32) (end 160.34 76.32) (width 0.2) (layer "B.Cu") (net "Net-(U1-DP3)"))
 (segment (start 138.75 78.245) (end 138.75 77.25) (width 0.2) (layer "F.Cu") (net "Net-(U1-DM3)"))
 (segment (start 138.75 77.25) (end 139.745 76.255) (width 0.2) (layer "F.Cu") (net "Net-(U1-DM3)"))
 (segment (start 155.18 74.47) (end 155.135 74.425) (width 0.2) (layer "F.Cu") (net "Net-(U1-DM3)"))
 (segment (start 139.745 76.255) (end 141.269571 76.255) (width 0.2) (layer "F.Cu") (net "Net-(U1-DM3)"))
 (segment (start 138.75 77.56259) (end 138.48241 77.295) (width 0.2) (layer "F.Cu") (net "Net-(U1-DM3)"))
 (segment (start 137.75 77.56259) (end 137.75 78.245) (width 0.2) (layer "F.Cu") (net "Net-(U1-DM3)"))
 (segment (start 154.6675 74.47) (end 155.18 74.47) (width 0.2) (layer "F.Cu") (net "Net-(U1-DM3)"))
 (segment (start 141.269571 76.255) (end 144.449571 73.075) (width 0.2) (layer "F.Cu") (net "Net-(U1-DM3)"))
 (segment (start 138.01759 77.295) (end 137.75 77.56259) (width 0.2) (layer "F.Cu") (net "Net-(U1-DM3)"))
 (segment (start 144.449571 73.075) (end 153.2725 73.075) (width 0.2) (layer "F.Cu") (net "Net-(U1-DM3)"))
 (segment (start 153.2725 73.075) (end 154.6675 74.47) (width 0.2) (layer "F.Cu") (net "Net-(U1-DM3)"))
 (segment (start 138.75 78.245) (end 138.75 77.56259) (width 0.2) (layer "F.Cu") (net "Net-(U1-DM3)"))
 (segment (start 138.48241 77.295) (end 138.01759 77.295) (width 0.2) (layer "F.Cu") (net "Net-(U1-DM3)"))
 (segment (start 145.675 72.325) (end 146 72) (width 0.2) (layer "F.Cu") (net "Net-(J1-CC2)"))
 (segment (start 136.25 77.56259) (end 136.25 78.245) (width 0.2) (layer "F.Cu") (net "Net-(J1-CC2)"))
 (segment (start 141.48759 72.325) (end 145.675 72.325) (width 0.2) (layer "F.Cu") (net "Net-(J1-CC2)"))
 (segment (start 146 72) (end 148.5 72) (width 0.2) (layer "F.Cu") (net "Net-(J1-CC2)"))
 (segment (start 141.48759 72.325) (end 136.25 77.56259) (width 0.2) (layer "F.Cu") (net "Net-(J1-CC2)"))
 (segment (start 133.68 77.605) (end 133.68 78.181237) (width 0.2) (layer "B.Cu") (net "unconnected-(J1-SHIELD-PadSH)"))
 (segment (start 142.32 73.425) (end 133.68 73.425) (width 0.2) (layer "B.Cu") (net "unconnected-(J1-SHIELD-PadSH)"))
 (segment (start 142.32 78.340685) (end 142.32 77.605) (width 0.2) (layer "B.Cu") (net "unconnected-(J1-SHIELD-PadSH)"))
 (segment (start 133.68 73.425) (end 133.68 77.605) (width 0.2) (layer "B.Cu") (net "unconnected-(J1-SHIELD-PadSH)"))
 (segment (start 133.68 78.181237) (end 135.093763 79.595) (width 0.2) (layer "B.Cu") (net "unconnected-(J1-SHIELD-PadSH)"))
 (segment (start 141.065685 79.595) (end 142.32 78.340685) (width 0.2) (layer "B.Cu") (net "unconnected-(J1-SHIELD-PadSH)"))
 (segment (start 135.093763 79.595) (end 141.065685 79.595) (width 0.2) (layer "B.Cu") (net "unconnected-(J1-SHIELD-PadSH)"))
 (segment (start 139.5 94.955) (end 138.5175 95.9375) (width 0.2) (layer "F.Cu") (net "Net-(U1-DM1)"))
 (segment (start 139.5 89.049571) (end 139.5 94.955) (width 0.2) (layer "F.Cu") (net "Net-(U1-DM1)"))
 (segment (start 155.18 79.54) (end 149.009571 79.54) (width 0.2) (layer "F.Cu") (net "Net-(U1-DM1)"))
 (segment (start 149.009571 79.54) (end 139.5 89.049571) (width 0.2) (layer "F.Cu") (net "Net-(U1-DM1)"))
 (segment (start 154.347256 78.96) (end 138.5175 94.789756) (width 0.2) (layer "B.Cu") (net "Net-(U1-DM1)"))
 (segment (start 138.5175 94.789756) (end 138.5175 95.9375) (width 0.2) (layer "B.Cu") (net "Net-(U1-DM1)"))
 (segment (start 160.92 79.54) (end 160.34 78.96) (width 0.2) (layer "B.Cu") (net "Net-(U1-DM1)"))
 (segment (start 160.34 78.96) (end 154.347256 78.96) (width 0.2) (layer "B.Cu") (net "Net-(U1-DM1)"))
 (segment (start 148.295256 80.82) (end 139.9 89.215256) (width 0.2) (layer "F.Cu") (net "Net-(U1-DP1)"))
 (segment (start 155.18 80.82) (end 148.295256 80.82) (width 0.2) (layer "F.Cu") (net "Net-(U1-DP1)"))
 (segment (start 139.9 89.215256) (end 139.9 95.32) (width 0.2) (layer "F.Cu") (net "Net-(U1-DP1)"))
 (segment (start 139.9 95.32) (end 140.5175 95.9375) (width 0.2) (layer "F.Cu") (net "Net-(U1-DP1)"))
 (segment (start 165.4375 81.75) (end 165.5 81.75) (width 0.2) (layer "F.Cu") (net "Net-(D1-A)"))
 (segment (start 161.1875 86) (end 165.4375 81.75) (width 0.2) (layer "F.Cu") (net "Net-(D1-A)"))
 (segment (start 155.18 77) (end 147.94957 77) (width 0.2) (layer "F.Cu") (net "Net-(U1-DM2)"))
 (segment (start 117.289815 97.3995) (end 123.057395 97.3995) (width 0.2) (layer "F.Cu") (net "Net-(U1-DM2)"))
 (segment (start 124.0795 96.377395) (end 124.0795 95.497605) (width 0.2) (layer "F.Cu") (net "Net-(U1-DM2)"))
 (segment (start 122.0795 94.8755) (end 121.0175 95.9375) (width 0.2) (layer "F.Cu") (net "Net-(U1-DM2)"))
 (segment (start 123.457395 94.8755) (end 122.0795 94.8755) (width 0.2) (layer "F.Cu") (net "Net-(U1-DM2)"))
 (segment (start 119.24957 88.5) (end 117.0555 90.694071) (width 0.2) (layer "F.Cu") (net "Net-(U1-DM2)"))
 (segment (start 117.0555 90.694071) (end 117.0555 97.165185) (width 0.2) (layer "F.Cu") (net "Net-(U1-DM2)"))
 (segment (start 123.057395 97.3995) (end 124.0795 96.377395) (width 0.2) (layer "F.Cu") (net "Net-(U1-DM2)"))
 (segment (start 147.94957 77) (end 136.44957 88.5) (width 0.2) (layer "F.Cu") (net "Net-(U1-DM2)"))
 (segment (start 124.0795 95.497605) (end 123.457395 94.8755) (width 0.2) (layer "F.Cu") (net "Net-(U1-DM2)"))
 (segment (start 117.0555 97.165185) (end 117.289815 97.3995) (width 0.2) (layer "F.Cu") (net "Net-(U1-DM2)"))
 (segment (start 136.44957 88.5) (end 119.24957 88.5) (width 0.2) (layer "F.Cu") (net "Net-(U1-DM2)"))
 (segment (start 147.245256 78.27) (end 136.615256 88.9) (width 0.2) (layer "F.Cu") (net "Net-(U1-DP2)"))
 (segment (start 117.4555 90.859756) (end 117.4555 96.9995) (width 0.2) (layer "F.Cu") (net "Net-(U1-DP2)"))
 (segment (start 155.18 78.27) (end 147.245256 78.27) (width 0.2) (layer "F.Cu") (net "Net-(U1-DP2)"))
 (segment (start 117.4555 96.9995) (end 121.9555 96.9995) (width 0.2) (layer "F.Cu") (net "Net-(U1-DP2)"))
 (segment (start 136.615256 88.9) (end 119.415256 88.9) (width 0.2) (layer "F.Cu") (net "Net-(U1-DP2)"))
 (segment (start 121.9555 96.9995) (end 123.0175 95.9375) (width 0.2) (layer "F.Cu") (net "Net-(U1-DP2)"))
 (segment (start 119.415256 88.9) (end 117.4555 90.859756) (width 0.2) (layer "F.Cu") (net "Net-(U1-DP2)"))
 (segment (start 123.0175 90.433971) (end 123.0175 95.9375) (width 0.2) (layer "B.Cu") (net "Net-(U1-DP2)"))
 (segment (start 124.051471 89.4) (end 123.0175 90.433971) (width 0.2) (layer "B.Cu") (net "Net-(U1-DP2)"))
 (segment (start 160.34 77.69) (end 153.699314 77.69) (width 0.2) (layer "B.Cu") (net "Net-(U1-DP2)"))
 (segment (start 153.699314 77.69) (end 141.989314 89.4) (width 0.2) (layer "B.Cu") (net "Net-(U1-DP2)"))
 (segment (start 160.92 78.27) (end 160.34 77.69) (width 0.2) (layer "B.Cu") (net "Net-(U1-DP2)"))
 (segment (start 141.989314 89.4) (end 124.051471 89.4) (width 0.2) (layer "B.Cu") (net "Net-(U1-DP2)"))
 (segment (start 166.6 83.15) (end 165.5 84.25) (width 0.2) (layer "F.Cu") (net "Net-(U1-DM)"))
 (segment (start 166.6 80.65) (end 166.6 83.15) (width 0.2) (layer "F.Cu") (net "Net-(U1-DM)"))
 (segment (start 160.92 80.82) (end 161.09 80.65) (width 0.2) (layer "F.Cu") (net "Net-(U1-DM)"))
 (segment (start 161.09 80.65) (end 166.6 80.65) (width 0.2) (layer "F.Cu") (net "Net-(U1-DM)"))
 (segment (start 159.7475 87.557244) (end 160.365256 88.175) (width 0.2) (layer "F.Cu") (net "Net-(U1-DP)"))
 (segment (start 160.365256 88.175) (end 163.575 88.175) (width 0.2) (layer "F.Cu") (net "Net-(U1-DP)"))
 (segment (start 163.575 88.175) (end 165.5 86.25) (width 0.2) (layer "F.Cu") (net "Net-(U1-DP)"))
 (segment (start 160.92 79.54) (end 160.4075 79.54) (width 0.2) (layer "F.Cu") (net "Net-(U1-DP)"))
 (segment (start 160.4075 79.54) (end 159.7475 80.2) (width 0.2) (layer "F.Cu") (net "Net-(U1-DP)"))
 (segment (start 159.7475 80.2) (end 159.7475 87.557244) (width 0.2) (layer "F.Cu") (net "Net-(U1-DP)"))
 (segment (start 164.937256 86.25) (end 165.5 86.25) (width 0.2) (layer "B.Cu") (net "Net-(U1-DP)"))
 (segment (start 158.227256 79.54) (end 164.937256 86.25) (width 0.2) (layer "B.Cu") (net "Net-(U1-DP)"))
 (segment (start 155.18 79.54) (end 158.227256 79.54) (width 0.2) (layer "B.Cu") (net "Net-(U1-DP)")))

